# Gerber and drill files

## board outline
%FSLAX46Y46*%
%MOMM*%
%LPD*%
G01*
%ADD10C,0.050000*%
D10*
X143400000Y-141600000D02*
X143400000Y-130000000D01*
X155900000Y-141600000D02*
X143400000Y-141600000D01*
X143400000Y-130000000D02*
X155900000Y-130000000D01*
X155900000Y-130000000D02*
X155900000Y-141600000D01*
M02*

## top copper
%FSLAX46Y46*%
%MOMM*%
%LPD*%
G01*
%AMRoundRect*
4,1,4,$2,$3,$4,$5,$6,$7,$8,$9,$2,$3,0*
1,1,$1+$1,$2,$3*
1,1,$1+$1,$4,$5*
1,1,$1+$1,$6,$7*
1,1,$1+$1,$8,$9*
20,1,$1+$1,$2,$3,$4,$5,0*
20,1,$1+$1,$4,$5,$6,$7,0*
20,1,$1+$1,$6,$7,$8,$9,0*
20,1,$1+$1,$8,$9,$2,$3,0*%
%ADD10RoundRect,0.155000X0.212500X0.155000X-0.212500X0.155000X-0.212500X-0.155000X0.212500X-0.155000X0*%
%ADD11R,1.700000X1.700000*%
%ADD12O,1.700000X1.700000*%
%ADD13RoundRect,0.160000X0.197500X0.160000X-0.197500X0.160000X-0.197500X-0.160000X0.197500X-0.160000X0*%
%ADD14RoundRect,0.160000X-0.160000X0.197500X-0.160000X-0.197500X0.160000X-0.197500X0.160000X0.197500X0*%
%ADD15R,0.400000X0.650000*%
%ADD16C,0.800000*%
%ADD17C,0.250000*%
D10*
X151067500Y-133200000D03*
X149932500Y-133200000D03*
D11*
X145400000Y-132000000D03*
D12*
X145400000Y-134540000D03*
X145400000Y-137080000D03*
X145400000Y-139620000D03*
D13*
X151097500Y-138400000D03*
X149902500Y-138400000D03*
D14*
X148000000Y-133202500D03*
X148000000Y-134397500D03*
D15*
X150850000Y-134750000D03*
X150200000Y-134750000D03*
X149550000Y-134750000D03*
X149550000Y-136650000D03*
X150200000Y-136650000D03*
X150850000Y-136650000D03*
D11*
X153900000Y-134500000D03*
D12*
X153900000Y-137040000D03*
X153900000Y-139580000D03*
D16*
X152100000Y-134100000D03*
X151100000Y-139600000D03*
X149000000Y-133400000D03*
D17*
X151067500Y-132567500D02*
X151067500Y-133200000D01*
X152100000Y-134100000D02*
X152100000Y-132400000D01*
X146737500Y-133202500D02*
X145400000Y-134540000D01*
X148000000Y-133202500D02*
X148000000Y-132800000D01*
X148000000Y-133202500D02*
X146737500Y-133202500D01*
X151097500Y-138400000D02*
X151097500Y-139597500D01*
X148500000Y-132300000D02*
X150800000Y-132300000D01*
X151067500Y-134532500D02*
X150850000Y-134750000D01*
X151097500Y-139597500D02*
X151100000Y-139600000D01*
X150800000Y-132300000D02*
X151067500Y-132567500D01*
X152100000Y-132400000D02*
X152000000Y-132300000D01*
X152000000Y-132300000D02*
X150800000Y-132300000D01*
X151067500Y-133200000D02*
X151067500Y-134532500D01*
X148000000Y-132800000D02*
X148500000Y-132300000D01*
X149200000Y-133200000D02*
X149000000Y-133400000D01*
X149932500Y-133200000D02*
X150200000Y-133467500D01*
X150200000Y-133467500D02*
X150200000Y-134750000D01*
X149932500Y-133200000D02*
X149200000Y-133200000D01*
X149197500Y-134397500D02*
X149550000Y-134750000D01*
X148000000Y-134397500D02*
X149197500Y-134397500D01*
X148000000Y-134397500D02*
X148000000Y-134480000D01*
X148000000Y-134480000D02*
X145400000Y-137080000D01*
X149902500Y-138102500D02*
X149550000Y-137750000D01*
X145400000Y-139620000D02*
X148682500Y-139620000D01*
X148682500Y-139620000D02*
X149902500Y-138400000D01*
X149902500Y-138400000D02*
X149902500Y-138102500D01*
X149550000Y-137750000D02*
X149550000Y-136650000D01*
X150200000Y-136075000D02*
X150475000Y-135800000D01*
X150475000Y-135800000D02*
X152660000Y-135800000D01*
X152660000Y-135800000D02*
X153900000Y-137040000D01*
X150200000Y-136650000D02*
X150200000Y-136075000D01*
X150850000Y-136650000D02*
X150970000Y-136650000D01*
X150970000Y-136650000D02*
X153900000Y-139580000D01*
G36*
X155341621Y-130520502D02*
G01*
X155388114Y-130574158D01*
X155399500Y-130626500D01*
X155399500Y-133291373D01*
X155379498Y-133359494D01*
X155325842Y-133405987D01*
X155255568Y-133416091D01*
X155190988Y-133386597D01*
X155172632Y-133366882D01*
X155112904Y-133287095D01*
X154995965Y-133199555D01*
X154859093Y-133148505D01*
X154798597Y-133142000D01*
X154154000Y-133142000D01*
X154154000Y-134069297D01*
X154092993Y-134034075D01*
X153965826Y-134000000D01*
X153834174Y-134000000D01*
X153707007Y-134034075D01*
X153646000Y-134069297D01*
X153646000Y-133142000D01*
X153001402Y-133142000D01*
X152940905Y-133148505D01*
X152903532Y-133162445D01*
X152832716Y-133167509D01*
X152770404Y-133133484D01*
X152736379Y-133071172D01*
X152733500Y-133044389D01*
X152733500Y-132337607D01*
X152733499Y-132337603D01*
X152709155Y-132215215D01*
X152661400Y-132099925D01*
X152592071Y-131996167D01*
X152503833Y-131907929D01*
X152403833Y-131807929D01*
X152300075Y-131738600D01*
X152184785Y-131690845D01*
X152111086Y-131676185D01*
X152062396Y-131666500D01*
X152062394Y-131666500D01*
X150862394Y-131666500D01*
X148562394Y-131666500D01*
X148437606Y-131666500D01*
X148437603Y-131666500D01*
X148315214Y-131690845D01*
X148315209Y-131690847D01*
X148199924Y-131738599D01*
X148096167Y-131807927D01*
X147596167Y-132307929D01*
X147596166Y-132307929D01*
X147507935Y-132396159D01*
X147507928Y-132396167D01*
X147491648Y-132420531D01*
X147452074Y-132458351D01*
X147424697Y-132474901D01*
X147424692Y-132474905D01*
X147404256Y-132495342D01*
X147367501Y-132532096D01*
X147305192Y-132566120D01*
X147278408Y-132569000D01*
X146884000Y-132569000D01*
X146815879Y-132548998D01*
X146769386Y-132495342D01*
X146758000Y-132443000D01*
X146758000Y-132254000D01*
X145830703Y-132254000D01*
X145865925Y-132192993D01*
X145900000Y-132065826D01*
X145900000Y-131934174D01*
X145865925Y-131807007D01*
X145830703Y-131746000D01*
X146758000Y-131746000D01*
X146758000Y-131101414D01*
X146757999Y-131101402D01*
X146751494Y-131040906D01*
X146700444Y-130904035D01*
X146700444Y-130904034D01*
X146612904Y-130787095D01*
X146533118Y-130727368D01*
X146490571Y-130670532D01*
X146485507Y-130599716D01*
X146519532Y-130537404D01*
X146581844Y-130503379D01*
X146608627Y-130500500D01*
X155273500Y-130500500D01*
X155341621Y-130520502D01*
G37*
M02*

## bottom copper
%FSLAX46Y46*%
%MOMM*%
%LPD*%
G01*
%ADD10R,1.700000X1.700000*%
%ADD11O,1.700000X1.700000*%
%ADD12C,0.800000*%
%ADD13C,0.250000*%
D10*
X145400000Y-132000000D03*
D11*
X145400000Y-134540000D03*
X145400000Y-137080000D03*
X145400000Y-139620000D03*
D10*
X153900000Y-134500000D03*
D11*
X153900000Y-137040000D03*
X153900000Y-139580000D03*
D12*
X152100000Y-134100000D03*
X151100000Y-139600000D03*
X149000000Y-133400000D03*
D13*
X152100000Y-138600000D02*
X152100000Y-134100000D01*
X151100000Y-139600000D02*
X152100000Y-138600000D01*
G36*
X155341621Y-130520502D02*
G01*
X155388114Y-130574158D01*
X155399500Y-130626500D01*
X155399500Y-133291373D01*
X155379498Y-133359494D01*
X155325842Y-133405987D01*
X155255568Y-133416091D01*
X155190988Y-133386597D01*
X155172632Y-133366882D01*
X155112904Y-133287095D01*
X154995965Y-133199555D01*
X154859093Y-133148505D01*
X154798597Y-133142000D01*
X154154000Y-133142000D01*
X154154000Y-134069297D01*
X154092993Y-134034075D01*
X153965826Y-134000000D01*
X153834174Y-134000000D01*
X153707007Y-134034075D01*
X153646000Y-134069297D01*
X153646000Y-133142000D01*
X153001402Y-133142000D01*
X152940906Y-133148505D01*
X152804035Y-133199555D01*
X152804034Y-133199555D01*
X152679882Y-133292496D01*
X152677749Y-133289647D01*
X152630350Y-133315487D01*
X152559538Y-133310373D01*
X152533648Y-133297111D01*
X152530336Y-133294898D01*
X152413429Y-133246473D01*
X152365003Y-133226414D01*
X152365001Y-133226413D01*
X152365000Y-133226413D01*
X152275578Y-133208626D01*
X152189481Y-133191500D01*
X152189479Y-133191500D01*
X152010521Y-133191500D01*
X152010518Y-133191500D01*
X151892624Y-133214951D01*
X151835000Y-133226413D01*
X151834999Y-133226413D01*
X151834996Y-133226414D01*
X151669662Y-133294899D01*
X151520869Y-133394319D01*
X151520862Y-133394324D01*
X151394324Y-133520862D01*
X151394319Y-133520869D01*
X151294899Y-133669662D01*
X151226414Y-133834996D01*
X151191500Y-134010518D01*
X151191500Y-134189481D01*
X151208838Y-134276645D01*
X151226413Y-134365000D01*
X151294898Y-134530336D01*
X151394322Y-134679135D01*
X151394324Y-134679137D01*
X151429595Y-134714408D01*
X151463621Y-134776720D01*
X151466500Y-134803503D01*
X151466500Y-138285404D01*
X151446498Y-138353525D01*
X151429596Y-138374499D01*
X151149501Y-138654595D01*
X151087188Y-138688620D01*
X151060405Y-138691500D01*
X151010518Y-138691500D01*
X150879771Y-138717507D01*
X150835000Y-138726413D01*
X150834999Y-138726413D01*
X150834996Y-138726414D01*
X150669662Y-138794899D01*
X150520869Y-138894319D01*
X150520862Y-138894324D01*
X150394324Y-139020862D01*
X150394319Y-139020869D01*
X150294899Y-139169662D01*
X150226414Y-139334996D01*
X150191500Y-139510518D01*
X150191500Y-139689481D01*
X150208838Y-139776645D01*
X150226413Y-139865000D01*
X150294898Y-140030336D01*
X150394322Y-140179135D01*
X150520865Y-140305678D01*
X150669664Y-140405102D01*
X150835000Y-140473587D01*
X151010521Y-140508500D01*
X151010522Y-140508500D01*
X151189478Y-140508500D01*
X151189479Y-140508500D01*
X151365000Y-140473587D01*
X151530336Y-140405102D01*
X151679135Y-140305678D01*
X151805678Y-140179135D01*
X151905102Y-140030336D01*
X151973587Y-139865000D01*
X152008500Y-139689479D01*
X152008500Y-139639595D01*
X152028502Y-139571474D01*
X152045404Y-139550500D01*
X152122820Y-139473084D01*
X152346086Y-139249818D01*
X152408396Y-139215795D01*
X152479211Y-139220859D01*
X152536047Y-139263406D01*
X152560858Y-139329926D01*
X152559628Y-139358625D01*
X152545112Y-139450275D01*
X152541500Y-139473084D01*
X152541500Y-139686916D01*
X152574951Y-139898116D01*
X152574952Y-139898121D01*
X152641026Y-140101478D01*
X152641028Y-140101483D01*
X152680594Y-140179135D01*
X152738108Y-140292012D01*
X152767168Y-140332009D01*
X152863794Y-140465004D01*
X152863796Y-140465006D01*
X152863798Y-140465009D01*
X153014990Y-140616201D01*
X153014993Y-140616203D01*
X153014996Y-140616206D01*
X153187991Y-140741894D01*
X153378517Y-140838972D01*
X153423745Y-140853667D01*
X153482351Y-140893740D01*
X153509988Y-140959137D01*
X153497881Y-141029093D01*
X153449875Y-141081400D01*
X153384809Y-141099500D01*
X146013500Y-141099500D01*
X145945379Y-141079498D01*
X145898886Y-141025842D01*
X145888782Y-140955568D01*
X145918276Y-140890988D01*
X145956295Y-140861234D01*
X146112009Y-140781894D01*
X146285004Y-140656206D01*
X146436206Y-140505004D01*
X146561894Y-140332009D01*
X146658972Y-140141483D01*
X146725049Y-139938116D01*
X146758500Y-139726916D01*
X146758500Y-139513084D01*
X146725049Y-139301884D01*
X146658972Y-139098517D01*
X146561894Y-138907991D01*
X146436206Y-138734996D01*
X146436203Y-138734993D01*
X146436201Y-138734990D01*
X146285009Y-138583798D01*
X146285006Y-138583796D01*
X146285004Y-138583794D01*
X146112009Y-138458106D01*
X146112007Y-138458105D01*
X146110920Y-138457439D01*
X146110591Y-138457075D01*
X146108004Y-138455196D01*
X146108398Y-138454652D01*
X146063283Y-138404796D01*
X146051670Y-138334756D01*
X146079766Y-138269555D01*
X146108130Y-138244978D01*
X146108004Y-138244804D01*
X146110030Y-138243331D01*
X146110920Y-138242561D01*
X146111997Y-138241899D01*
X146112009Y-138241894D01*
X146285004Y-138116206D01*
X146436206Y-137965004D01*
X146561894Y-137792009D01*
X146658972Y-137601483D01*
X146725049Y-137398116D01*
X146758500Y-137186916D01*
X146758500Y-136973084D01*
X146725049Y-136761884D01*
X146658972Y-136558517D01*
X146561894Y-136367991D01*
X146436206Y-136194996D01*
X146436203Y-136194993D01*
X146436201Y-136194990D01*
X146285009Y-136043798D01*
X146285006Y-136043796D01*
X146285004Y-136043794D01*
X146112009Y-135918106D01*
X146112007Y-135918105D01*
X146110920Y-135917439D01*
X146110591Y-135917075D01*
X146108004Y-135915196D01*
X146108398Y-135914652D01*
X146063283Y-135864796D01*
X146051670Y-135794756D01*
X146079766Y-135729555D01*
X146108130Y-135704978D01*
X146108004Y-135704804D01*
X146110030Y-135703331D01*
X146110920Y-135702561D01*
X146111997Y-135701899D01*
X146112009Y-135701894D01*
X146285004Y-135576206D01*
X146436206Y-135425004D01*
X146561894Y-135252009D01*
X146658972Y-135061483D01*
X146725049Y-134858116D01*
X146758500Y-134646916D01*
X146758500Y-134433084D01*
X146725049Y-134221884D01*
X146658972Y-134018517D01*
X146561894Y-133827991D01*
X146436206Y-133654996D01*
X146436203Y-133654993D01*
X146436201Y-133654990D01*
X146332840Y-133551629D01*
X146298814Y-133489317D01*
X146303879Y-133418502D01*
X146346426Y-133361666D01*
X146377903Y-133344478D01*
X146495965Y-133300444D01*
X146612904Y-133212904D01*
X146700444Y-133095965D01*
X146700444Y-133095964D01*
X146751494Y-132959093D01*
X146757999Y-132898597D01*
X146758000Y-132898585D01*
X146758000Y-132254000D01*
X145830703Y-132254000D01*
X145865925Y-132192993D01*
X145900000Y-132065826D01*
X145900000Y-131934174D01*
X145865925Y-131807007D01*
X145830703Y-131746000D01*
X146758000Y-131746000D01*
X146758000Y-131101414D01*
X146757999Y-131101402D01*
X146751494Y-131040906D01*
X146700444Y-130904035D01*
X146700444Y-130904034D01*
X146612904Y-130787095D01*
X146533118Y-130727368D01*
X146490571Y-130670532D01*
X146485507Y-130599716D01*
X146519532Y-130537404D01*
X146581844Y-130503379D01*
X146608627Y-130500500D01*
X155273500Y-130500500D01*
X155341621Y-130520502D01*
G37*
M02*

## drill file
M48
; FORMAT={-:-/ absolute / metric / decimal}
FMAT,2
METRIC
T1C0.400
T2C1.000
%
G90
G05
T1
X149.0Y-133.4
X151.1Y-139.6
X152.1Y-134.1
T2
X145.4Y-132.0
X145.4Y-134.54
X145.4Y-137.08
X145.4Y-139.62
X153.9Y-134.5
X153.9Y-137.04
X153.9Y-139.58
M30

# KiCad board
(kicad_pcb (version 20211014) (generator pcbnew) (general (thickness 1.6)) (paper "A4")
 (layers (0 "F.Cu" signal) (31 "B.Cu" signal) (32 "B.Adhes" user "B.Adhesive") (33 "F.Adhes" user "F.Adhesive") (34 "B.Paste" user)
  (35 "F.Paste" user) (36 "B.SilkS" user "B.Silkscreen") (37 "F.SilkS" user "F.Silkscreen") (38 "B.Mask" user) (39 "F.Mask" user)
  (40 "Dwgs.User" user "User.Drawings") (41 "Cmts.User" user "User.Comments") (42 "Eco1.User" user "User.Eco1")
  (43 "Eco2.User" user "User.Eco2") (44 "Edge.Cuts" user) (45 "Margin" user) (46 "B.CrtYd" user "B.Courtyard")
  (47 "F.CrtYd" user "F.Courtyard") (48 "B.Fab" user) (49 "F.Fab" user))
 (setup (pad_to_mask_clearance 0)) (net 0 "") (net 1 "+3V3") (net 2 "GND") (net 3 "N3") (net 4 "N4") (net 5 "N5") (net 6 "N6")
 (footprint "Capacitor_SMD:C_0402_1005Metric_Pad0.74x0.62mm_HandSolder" (layer "F.Cu") (at 150.5 133.2 180)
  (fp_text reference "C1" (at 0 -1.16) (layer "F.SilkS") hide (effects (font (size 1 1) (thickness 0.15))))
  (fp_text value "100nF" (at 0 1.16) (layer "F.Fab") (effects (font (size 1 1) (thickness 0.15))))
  (pad "1" smd roundrect locked (at -0.5675 0 180) (size 0.735 0.62) (layers "F.Cu" "F.Paste" "F.Mask") (roundrect_rratio 0.25)
   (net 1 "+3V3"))
  (pad "2" smd roundrect locked (at 0.5675 0 180) (size 0.735 0.62) (layers "F.Cu" "F.Paste" "F.Mask") (roundrect_rratio 0.25) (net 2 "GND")))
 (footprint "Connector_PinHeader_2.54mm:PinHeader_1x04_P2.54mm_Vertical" (layer "F.Cu") (at 145.4 132)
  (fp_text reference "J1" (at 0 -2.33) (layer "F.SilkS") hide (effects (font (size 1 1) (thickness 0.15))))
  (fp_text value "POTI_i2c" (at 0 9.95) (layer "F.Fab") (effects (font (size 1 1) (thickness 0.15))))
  (pad "1" thru_hole rect locked (at 0 0) (size 1.7 1.7) (drill 1) (layers *.Cu *.Mask) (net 2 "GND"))
  (pad "2" thru_hole oval locked (at 0 2.54) (size 1.7 1.7) (drill 1) (layers *.Cu *.Mask) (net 1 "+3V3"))
  (pad "3" thru_hole oval locked (at 0 5.08) (size 1.7 1.7) (drill 1) (layers *.Cu *.Mask) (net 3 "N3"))
  (pad "4" thru_hole oval locked (at 0 7.62) (size 1.7 1.7) (drill 1) (layers *.Cu *.Mask) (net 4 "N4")))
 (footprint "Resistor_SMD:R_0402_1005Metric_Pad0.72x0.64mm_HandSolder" (layer "F.Cu") (at 150.5 138.4 180)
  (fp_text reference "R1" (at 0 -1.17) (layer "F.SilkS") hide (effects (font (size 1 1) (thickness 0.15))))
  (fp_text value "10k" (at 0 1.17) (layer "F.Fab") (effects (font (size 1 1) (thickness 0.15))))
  (pad "1" smd roundrect locked (at -0.5975 0 180) (size 0.715 0.64) (layers "F.Cu" "F.Paste" "F.Mask") (roundrect_rratio 0.25)
   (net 1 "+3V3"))
  (pad "2" smd roundrect locked (at 0.5975 0 180) (size 0.715 0.64) (layers "F.Cu" "F.Paste" "F.Mask") (roundrect_rratio 0.25) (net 4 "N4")))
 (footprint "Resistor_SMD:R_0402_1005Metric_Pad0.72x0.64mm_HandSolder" (layer "F.Cu") (at 148 133.8 -90)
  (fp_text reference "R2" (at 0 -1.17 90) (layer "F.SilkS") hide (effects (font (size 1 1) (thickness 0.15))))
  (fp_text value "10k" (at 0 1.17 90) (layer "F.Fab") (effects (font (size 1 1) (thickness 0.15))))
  (pad "1" smd roundrect locked (at -0.5975 0 270) (size 0.715 0.64) (layers "F.Cu" "F.Paste" "F.Mask") (roundrect_rratio 0.25)
   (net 1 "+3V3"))
  (pad "2" smd roundrect locked (at 0.5975 0 270) (size 0.715 0.64) (layers "F.Cu" "F.Paste" "F.Mask") (roundrect_rratio 0.25) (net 3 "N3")))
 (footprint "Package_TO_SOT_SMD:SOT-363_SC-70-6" (layer "F.Cu") (at 150.2 135.7 -90)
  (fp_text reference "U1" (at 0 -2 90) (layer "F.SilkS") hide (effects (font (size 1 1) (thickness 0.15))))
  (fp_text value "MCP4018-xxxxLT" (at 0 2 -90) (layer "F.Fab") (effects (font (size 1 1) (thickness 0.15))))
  (pad "1" smd rect locked (at -0.95 -0.65 270) (size 0.65 0.4) (layers "F.Cu" "F.Paste" "F.Mask") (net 1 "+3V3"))
  (pad "2" smd rect locked (at -0.95 0 270) (size 0.65 0.4) (layers "F.Cu" "F.Paste" "F.Mask") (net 2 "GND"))
  (pad "3" smd rect locked (at -0.95 0.65 270) (size 0.65 0.4) (layers "F.Cu" "F.Paste" "F.Mask") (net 3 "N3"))
  (pad "4" smd rect locked (at 0.95 0.65 270) (size 0.65 0.4) (layers "F.Cu" "F.Paste" "F.Mask") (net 4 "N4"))
  (pad "5" smd rect locked (at 0.95 0 270) (size 0.65 0.4) (layers "F.Cu" "F.Paste" "F.Mask") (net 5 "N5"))
  (pad "6" smd rect locked (at 0.95 -0.65 270) (size 0.65 0.4) (layers "F.Cu" "F.Paste" "F.Mask") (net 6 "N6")))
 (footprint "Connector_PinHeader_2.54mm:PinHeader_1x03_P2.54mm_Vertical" (layer "B.Cu") (at 153.9 134.5 180)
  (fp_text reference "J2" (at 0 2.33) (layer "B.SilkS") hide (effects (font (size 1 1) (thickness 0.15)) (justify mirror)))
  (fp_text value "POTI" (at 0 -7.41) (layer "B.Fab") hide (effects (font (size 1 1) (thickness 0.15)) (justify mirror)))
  (pad "1" thru_hole rect locked (at 0 0 180) (size 1.7 1.7) (drill 1) (layers *.Cu *.Mask) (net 2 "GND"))
  (pad "2" thru_hole oval locked (at 0 -2.54 180) (size 1.7 1.7) (drill 1) (layers *.Cu *.Mask) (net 5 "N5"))
  (pad "3" thru_hole oval locked (at 0 -5.08 180) (size 1.7 1.7) (drill 1) (layers *.Cu *.Mask) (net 6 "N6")))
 (gr_line (start 143.4 141.6) (end 143.4 130) (layer "Edge.Cuts") (width 0.05))
 (gr_line (start 155.9 141.6) (end 143.4 141.6) (layer "Edge.Cuts") (width 0.05))
 (gr_line (start 143.4 130) (end 155.9 130) (layer "Edge.Cuts") (width 0.05))
 (gr_line (start 155.9 130) (end 155.9 141.6) (layer "Edge.Cuts") (width 0.05))
 (segment (start 151.0675 132.5675) (end 151.0675 133.2) (width 0.25) (layer "F.Cu") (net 1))
 (segment (start 152.1 134.1) (end 152.1 132.4) (width 0.25) (layer "F.Cu") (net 1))
 (segment (start 146.7375 133.2025) (end 145.4 134.54) (width 0.25) (layer "F.Cu") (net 1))
 (segment (start 148 133.2025) (end 148 132.8) (width 0.25) (layer "F.Cu") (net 1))
 (segment (start 148 133.2025) (end 146.7375 133.2025) (width 0.25) (layer "F.Cu") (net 1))
 (segment (start 151.0975 138.4) (end 151.0975 139.5975) (width 0.25) (layer "F.Cu") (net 1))
 (segment (start 148.5 132.3) (end 150.8 132.3) (width 0.25) (layer "F.Cu") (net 1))
 (segment (start 151.0675 134.5325) (end 150.85 134.75) (width 0.25) (layer "F.Cu") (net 1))
 (segment (start 151.0975 139.5975) (end 151.1 139.6) (width 0.25) (layer "F.Cu") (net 1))
 (segment (start 150.8 132.3) (end 151.0675 132.5675) (width 0.25) (layer "F.Cu") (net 1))
 (segment (start 152.1 132.4) (end 152 132.3) (width 0.25) (layer "F.Cu") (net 1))
 (segment (start 152 132.3) (end 150.8 132.3) (width 0.25) (layer "F.Cu") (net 1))
 (segment (start 151.0675 133.2) (end 151.0675 134.5325) (width 0.25) (layer "F.Cu") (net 1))
 (segment (start 148 132.8) (end 148.5 132.3) (width 0.25) (layer "F.Cu") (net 1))
 (via (at 152.1 134.1) (size 0.8) (drill 0.4) (layers "F.Cu" "B.Cu") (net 1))
 (via (at 151.1 139.6) (size 0.8) (drill 0.4) (layers "F.Cu" "B.Cu") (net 1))
 (segment (start 152.1 138.6) (end 152.1 134.1) (width 0.25) (layer "B.Cu") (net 1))
 (segment (start 151.1 139.6) (end 152.1 138.6) (width 0.25) (layer "B.Cu") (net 1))
 (segment (start 149.2 133.2) (end 149 133.4) (width 0.25) (layer "F.Cu") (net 2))
 (segment (start 149.9325 133.2) (end 150.2 133.4675) (width 0.25) (layer "F.Cu") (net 2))
 (segment (start 150.2 133.4675) (end 150.2 134.75) (width 0.25) (layer "F.Cu") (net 2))
 (segment (start 149.9325 133.2) (end 149.2 133.2) (width 0.25) (layer "F.Cu") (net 2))
 (via (at 149 133.4) (size 0.8) (drill 0.4) (layers "F.Cu" "B.Cu") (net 2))
 (segment (start 149.1975 134.3975) (end 149.55 134.75) (width 0.25) (layer "F.Cu") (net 3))
 (segment (start 148 134.3975) (end 149.1975 134.3975) (width 0.25) (layer "F.Cu") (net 3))
 (segment (start 148 134.3975) (end 148 134.48) (width 0.25) (layer "F.Cu") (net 3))
 (segment (start 148 134.48) (end 145.4 137.08) (width 0.25) (layer "F.Cu") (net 3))
 (segment (start 149.9025 138.1025) (end 149.55 137.75) (width 0.25) (layer "F.Cu") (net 4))
 (segment (start 145.4 139.62) (end 148.6825 139.62) (width 0.25) (layer "F.Cu") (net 4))
 (segment (start 148.6825 139.62) (end 149.9025 138.4) (width 0.25) (layer "F.Cu") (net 4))
 (segment (start 149.9025 138.4) (end 149.9025 138.1025) (width 0.25) (layer "F.Cu") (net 4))
 (segment (start 149.55 137.75) (end 149.55 136.65) (width 0.25) (layer "F.Cu") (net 4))
 (segment (start 150.2 136.075) (end 150.475 135.8) (width 0.25) (layer "F.Cu") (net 5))
 (segment (start 150.475 135.8) (end 152.66 135.8) (width 0.25) (layer "F.Cu") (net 5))
 (segment (start 152.66 135.8) (end 153.9 137.04) (width 0.25) (layer "F.Cu") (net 5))
 (segment (start 150.2 136.65) (end 150.2 136.075) (width 0.25) (layer "F.Cu") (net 5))
 (segment (start 150.85 136.65) (end 150.97 136.65) (width 0.25) (layer "F.Cu") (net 6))
 (segment (start 150.97 136.65) (end 153.9 139.58) (width 0.25) (layer "F.Cu") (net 6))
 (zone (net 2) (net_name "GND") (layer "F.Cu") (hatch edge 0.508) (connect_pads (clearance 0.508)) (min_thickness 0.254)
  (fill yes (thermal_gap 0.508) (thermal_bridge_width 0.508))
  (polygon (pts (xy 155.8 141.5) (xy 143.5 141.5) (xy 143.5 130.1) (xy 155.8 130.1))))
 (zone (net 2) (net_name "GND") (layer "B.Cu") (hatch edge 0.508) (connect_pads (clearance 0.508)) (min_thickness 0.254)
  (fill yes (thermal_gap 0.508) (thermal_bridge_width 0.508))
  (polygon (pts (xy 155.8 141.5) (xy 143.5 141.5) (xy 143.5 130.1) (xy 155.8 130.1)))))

